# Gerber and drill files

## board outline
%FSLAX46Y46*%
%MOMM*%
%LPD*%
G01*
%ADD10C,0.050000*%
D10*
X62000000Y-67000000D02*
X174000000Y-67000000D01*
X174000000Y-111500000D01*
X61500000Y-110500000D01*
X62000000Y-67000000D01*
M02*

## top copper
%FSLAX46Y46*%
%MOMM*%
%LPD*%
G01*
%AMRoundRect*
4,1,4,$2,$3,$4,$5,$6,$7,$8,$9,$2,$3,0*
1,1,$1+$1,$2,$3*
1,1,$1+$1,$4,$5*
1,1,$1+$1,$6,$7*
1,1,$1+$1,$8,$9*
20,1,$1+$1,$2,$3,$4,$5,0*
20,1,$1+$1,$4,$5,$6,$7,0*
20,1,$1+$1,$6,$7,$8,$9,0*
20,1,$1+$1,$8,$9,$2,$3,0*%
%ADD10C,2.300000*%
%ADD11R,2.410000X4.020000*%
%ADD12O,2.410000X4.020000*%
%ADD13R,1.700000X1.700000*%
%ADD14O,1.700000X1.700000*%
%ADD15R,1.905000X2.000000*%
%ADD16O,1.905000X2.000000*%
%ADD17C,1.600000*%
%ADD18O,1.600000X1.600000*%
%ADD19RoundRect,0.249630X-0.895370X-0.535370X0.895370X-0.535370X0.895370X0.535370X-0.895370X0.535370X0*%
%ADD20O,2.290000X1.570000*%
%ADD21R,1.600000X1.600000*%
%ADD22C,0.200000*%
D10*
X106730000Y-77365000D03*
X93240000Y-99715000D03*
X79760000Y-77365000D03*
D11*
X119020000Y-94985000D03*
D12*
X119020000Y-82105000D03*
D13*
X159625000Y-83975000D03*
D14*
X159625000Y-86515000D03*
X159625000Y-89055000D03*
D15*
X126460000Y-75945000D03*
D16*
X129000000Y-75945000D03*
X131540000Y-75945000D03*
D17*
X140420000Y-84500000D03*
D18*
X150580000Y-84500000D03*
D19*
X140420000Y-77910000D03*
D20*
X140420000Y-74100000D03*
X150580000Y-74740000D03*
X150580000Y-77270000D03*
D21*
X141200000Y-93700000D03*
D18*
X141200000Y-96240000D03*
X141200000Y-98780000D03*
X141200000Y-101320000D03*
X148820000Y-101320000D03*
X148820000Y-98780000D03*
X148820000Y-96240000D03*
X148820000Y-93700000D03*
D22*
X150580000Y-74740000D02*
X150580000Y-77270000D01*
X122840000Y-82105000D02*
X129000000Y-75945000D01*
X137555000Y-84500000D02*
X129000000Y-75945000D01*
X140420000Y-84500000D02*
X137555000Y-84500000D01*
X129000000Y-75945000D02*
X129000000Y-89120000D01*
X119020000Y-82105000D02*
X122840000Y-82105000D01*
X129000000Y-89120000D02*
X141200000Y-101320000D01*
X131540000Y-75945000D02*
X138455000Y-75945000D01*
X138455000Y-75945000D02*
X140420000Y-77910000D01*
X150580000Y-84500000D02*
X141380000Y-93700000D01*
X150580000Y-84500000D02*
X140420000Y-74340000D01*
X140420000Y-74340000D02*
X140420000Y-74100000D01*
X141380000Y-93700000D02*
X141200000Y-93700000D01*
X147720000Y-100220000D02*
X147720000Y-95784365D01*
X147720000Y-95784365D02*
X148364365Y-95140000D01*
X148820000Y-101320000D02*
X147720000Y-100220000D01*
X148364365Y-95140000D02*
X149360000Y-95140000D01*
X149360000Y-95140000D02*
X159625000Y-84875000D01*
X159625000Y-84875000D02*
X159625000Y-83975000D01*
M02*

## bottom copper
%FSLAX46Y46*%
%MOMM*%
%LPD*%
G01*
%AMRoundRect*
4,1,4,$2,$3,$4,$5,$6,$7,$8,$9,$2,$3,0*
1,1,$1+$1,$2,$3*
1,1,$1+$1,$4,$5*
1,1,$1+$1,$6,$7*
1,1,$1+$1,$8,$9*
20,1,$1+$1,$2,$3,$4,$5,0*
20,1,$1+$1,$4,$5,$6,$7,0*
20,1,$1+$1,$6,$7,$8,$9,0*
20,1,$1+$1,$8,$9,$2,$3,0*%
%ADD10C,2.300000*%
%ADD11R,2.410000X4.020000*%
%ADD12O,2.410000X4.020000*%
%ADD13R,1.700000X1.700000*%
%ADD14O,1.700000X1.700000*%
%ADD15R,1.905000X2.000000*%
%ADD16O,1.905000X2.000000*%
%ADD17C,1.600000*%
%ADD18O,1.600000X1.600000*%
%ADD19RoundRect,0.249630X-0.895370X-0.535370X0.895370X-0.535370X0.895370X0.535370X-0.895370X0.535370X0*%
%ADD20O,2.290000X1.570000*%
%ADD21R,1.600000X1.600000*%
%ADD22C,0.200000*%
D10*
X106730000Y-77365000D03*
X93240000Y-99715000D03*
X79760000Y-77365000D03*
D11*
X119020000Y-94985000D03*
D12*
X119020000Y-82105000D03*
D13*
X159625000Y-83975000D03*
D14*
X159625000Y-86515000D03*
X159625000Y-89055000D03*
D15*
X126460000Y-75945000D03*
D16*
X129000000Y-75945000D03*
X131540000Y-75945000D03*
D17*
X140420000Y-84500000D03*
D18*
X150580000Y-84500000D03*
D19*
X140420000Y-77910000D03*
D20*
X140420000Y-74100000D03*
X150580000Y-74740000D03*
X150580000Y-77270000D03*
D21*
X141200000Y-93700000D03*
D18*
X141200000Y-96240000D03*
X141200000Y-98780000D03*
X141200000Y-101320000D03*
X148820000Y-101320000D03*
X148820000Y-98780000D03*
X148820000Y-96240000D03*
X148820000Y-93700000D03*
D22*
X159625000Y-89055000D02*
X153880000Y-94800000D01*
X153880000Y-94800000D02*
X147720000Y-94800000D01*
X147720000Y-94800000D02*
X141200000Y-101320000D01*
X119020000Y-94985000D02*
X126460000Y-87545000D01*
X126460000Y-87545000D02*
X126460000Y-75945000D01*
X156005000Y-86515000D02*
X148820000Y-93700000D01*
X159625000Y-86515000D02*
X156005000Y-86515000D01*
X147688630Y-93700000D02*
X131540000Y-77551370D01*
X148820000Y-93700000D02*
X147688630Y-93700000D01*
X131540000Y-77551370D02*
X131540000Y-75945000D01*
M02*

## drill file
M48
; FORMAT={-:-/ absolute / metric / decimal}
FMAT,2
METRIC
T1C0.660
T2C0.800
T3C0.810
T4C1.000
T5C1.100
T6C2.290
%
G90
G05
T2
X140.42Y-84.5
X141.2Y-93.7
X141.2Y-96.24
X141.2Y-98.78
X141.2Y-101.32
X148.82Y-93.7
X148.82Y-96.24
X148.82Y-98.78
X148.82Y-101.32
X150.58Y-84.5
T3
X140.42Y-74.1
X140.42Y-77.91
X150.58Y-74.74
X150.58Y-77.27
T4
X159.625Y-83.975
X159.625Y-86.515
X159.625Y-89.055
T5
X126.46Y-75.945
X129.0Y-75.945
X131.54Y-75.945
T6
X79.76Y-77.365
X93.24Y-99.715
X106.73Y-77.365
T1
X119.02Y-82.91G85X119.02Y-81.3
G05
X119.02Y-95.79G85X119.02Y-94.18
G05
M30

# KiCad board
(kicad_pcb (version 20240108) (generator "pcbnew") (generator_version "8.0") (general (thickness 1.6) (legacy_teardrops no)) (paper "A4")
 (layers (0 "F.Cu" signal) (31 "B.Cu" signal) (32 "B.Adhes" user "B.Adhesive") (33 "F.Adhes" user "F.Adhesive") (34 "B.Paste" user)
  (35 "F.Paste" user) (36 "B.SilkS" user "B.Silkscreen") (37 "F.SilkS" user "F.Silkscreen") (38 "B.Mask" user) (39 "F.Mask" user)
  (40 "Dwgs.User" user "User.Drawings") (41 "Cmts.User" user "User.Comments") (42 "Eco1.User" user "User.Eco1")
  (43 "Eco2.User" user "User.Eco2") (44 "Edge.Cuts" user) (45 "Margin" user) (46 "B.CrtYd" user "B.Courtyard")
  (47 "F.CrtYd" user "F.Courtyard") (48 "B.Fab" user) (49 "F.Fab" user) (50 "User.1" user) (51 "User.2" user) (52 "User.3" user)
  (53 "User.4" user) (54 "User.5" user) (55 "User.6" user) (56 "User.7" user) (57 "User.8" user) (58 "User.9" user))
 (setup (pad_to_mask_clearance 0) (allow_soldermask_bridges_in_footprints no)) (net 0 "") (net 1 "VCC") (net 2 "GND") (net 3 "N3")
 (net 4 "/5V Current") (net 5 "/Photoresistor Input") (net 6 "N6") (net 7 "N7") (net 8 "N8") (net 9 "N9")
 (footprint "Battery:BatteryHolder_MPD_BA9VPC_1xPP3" (layer "F.Cu") (at 119.02 94.985 180)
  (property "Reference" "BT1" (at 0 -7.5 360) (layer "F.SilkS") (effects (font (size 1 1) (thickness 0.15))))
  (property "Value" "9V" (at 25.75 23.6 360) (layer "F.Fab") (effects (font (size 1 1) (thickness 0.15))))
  (pad "" np_thru_hole circle (at 12.29 17.62 180) (size 2.3 2.3) (drill 2.29) (layers "*.Cu" "*.Mask"))
  (pad "" np_thru_hole circle (at 25.78 -4.73 180) (size 2.3 2.3) (drill 2.29) (layers "*.Cu" "*.Mask"))
  (pad "" np_thru_hole circle (at 39.26 17.62 180) (size 2.3 2.3) (drill 2.29) (layers "*.Cu" "*.Mask"))
  (pad "1" thru_hole rect (at 0 0 180) (size 2.41 4.02) (drill oval 0.66 2.27) (layers "*.Cu" "*.Mask") (remove_unused_layers no)
   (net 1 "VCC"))
  (pad "2" thru_hole oval (at 0 12.88 180) (size 2.41 4.02) (drill oval 0.66 2.27) (layers "*.Cu" "*.Mask") (remove_unused_layers no)
   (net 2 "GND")))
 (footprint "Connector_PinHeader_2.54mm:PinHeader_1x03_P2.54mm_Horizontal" (layer "F.Cu") (at 159.625 83.975)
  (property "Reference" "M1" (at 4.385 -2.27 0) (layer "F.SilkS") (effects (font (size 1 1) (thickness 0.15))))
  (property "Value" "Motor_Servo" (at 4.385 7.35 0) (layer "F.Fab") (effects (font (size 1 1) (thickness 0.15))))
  (pad "1" thru_hole rect (at 0 0) (size 1.7 1.7) (drill 1) (layers "*.Cu" "*.Mask") (remove_unused_layers no) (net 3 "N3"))
  (pad "2" thru_hole oval (at 0 2.54) (size 1.7 1.7) (drill 1) (layers "*.Cu" "*.Mask") (remove_unused_layers no) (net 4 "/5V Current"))
  (pad "3" thru_hole oval (at 0 5.08) (size 1.7 1.7) (drill 1) (layers "*.Cu" "*.Mask") (remove_unused_layers no) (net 2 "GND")))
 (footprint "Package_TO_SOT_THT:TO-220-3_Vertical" (layer "F.Cu") (at 126.46 75.945)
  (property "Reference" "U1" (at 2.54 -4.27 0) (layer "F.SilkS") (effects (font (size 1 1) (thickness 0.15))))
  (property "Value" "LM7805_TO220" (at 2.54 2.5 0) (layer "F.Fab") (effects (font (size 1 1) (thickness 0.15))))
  (pad "1" thru_hole rect (at 0 0) (size 1.905 2) (drill 1.1) (layers "*.Cu" "*.Mask") (remove_unused_layers no) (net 1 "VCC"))
  (pad "2" thru_hole oval (at 2.54 0) (size 1.905 2) (drill 1.1) (layers "*.Cu" "*.Mask") (remove_unused_layers no) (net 2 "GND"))
  (pad "3" thru_hole oval (at 5.08 0) (size 1.905 2) (drill 1.1) (layers "*.Cu" "*.Mask") (remove_unused_layers no) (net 4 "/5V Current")))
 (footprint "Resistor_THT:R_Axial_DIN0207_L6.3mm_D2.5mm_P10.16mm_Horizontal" (layer "F.Cu") (at 140.42 84.5)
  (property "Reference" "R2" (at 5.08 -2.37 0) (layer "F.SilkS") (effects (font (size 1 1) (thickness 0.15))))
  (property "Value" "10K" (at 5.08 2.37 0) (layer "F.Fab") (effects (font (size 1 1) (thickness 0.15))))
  (pad "1" thru_hole circle (at 0 0) (size 1.6 1.6) (drill 0.8) (layers "*.Cu" "*.Mask") (remove_unused_layers no) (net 2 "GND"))
  (pad "2" thru_hole oval (at 10.16 0) (size 1.6 1.6) (drill 0.8) (layers "*.Cu" "*.Mask") (remove_unused_layers no)
   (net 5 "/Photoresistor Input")))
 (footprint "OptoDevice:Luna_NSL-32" (layer "F.Cu") (at 140.42 77.91)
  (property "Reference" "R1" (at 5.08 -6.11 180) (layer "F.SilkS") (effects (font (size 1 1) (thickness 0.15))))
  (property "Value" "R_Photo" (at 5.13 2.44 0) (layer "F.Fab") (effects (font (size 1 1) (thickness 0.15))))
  (pad "1" thru_hole roundrect (at 0 0) (size 2.29 1.57) (drill 0.81) (layers "*.Cu" "*.Mask") (remove_unused_layers no)
   (roundrect_rratio 0.159) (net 4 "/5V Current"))
  (pad "2" thru_hole oval (at 0 -3.81) (size 2.29 1.57) (drill 0.81) (layers "*.Cu" "*.Mask") (remove_unused_layers no)
   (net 5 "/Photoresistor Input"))
  (pad "3" thru_hole oval (at 10.16 -3.17) (size 2.29 1.57) (drill 0.81) (layers "*.Cu" "*.Mask") (remove_unused_layers no))
  (pad "4" thru_hole oval (at 10.16 -0.64) (size 2.29 1.57) (drill 0.81) (layers "*.Cu" "*.Mask") (remove_unused_layers no)))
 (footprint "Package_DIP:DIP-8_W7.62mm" (layer "F.Cu") (at 141.2 93.7)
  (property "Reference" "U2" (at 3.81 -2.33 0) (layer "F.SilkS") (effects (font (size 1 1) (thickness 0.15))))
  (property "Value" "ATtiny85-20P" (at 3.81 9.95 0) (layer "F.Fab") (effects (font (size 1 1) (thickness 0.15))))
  (pad "1" thru_hole rect (at 0 0) (size 1.6 1.6) (drill 0.8) (layers "*.Cu" "*.Mask") (remove_unused_layers no)
   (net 5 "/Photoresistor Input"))
  (pad "2" thru_hole oval (at 0 2.54) (size 1.6 1.6) (drill 0.8) (layers "*.Cu" "*.Mask") (remove_unused_layers no) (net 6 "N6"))
  (pad "3" thru_hole oval (at 0 5.08) (size 1.6 1.6) (drill 0.8) (layers "*.Cu" "*.Mask") (remove_unused_layers no) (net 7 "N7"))
  (pad "4" thru_hole oval (at 0 7.62) (size 1.6 1.6) (drill 0.8) (layers "*.Cu" "*.Mask") (remove_unused_layers no) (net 2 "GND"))
  (pad "5" thru_hole oval (at 7.62 7.62) (size 1.6 1.6) (drill 0.8) (layers "*.Cu" "*.Mask") (remove_unused_layers no) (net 3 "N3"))
  (pad "6" thru_hole oval (at 7.62 5.08) (size 1.6 1.6) (drill 0.8) (layers "*.Cu" "*.Mask") (remove_unused_layers no) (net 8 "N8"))
  (pad "7" thru_hole oval (at 7.62 2.54) (size 1.6 1.6) (drill 0.8) (layers "*.Cu" "*.Mask") (remove_unused_layers no) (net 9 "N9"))
  (pad "8" thru_hole oval (at 7.62 0) (size 1.6 1.6) (drill 0.8) (layers "*.Cu" "*.Mask") (remove_unused_layers no) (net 4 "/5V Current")))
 (gr_poly (pts (xy 62 67) (xy 174 67) (xy 174 111.5) (xy 61.5 110.5)) (stroke (width 0.05) (type solid)) (fill none) (layer "Edge.Cuts"))
 (segment (start 150.58 74.74) (end 150.58 77.27) (width 0.2) (layer "F.Cu") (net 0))
 (segment (start 122.84 82.105) (end 129 75.945) (width 0.2) (layer "F.Cu") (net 2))
 (segment (start 137.555 84.5) (end 129 75.945) (width 0.2) (layer "F.Cu") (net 2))
 (segment (start 140.42 84.5) (end 137.555 84.5) (width 0.2) (layer "F.Cu") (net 2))
 (segment (start 129 75.945) (end 129 89.12) (width 0.2) (layer "F.Cu") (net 2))
 (segment (start 119.02 82.105) (end 122.84 82.105) (width 0.2) (layer "F.Cu") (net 2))
 (segment (start 129 89.12) (end 141.2 101.32) (width 0.2) (layer "F.Cu") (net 2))
 (segment (start 159.625 89.055) (end 153.88 94.8) (width 0.2) (layer "B.Cu") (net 2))
 (segment (start 153.88 94.8) (end 147.72 94.8) (width 0.2) (layer "B.Cu") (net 2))
 (segment (start 147.72 94.8) (end 141.2 101.32) (width 0.2) (layer "B.Cu") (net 2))
 (segment (start 119.02 94.985) (end 126.46 87.545) (width 0.2) (layer "B.Cu") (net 1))
 (segment (start 126.46 87.545) (end 126.46 75.945) (width 0.2) (layer "B.Cu") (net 1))
 (segment (start 131.54 75.945) (end 138.455 75.945) (width 0.2) (layer "F.Cu") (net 4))
 (segment (start 138.455 75.945) (end 140.42 77.91) (width 0.2) (layer "F.Cu") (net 4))
 (segment (start 156.005 86.515) (end 148.82 93.7) (width 0.2) (layer "B.Cu") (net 4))
 (segment (start 159.625 86.515) (end 156.005 86.515) (width 0.2) (layer "B.Cu") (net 4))
 (segment (start 147.68863 93.7) (end 131.54 77.55137) (width 0.2) (layer "B.Cu") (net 4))
 (segment (start 148.82 93.7) (end 147.68863 93.7) (width 0.2) (layer "B.Cu") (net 4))
 (segment (start 131.54 77.55137) (end 131.54 75.945) (width 0.2) (layer "B.Cu") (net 4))
 (segment (start 150.58 84.5) (end 141.38 93.7) (width 0.2) (layer "F.Cu") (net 5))
 (segment (start 150.58 84.5) (end 140.42 74.34) (width 0.2) (layer "F.Cu") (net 5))
 (segment (start 140.42 74.34) (end 140.42 74.1) (width 0.2) (layer "F.Cu") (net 5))
 (segment (start 141.38 93.7) (end 141.2 93.7) (width 0.2) (layer "F.Cu") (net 5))
 (segment (start 147.72 100.22) (end 147.72 95.784365) (width 0.2) (layer "F.Cu") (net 3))
 (segment (start 147.72 95.784365) (end 148.364365 95.14) (width 0.2) (layer "F.Cu") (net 3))
 (segment (start 148.82 101.32) (end 147.72 100.22) (width 0.2) (layer "F.Cu") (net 3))
 (segment (start 148.364365 95.14) (end 149.36 95.14) (width 0.2) (layer "F.Cu") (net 3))
 (segment (start 149.36 95.14) (end 159.625 84.875) (width 0.2) (layer "F.Cu") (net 3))
 (segment (start 159.625 84.875) (end 159.625 83.975) (width 0.2) (layer "F.Cu") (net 3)))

